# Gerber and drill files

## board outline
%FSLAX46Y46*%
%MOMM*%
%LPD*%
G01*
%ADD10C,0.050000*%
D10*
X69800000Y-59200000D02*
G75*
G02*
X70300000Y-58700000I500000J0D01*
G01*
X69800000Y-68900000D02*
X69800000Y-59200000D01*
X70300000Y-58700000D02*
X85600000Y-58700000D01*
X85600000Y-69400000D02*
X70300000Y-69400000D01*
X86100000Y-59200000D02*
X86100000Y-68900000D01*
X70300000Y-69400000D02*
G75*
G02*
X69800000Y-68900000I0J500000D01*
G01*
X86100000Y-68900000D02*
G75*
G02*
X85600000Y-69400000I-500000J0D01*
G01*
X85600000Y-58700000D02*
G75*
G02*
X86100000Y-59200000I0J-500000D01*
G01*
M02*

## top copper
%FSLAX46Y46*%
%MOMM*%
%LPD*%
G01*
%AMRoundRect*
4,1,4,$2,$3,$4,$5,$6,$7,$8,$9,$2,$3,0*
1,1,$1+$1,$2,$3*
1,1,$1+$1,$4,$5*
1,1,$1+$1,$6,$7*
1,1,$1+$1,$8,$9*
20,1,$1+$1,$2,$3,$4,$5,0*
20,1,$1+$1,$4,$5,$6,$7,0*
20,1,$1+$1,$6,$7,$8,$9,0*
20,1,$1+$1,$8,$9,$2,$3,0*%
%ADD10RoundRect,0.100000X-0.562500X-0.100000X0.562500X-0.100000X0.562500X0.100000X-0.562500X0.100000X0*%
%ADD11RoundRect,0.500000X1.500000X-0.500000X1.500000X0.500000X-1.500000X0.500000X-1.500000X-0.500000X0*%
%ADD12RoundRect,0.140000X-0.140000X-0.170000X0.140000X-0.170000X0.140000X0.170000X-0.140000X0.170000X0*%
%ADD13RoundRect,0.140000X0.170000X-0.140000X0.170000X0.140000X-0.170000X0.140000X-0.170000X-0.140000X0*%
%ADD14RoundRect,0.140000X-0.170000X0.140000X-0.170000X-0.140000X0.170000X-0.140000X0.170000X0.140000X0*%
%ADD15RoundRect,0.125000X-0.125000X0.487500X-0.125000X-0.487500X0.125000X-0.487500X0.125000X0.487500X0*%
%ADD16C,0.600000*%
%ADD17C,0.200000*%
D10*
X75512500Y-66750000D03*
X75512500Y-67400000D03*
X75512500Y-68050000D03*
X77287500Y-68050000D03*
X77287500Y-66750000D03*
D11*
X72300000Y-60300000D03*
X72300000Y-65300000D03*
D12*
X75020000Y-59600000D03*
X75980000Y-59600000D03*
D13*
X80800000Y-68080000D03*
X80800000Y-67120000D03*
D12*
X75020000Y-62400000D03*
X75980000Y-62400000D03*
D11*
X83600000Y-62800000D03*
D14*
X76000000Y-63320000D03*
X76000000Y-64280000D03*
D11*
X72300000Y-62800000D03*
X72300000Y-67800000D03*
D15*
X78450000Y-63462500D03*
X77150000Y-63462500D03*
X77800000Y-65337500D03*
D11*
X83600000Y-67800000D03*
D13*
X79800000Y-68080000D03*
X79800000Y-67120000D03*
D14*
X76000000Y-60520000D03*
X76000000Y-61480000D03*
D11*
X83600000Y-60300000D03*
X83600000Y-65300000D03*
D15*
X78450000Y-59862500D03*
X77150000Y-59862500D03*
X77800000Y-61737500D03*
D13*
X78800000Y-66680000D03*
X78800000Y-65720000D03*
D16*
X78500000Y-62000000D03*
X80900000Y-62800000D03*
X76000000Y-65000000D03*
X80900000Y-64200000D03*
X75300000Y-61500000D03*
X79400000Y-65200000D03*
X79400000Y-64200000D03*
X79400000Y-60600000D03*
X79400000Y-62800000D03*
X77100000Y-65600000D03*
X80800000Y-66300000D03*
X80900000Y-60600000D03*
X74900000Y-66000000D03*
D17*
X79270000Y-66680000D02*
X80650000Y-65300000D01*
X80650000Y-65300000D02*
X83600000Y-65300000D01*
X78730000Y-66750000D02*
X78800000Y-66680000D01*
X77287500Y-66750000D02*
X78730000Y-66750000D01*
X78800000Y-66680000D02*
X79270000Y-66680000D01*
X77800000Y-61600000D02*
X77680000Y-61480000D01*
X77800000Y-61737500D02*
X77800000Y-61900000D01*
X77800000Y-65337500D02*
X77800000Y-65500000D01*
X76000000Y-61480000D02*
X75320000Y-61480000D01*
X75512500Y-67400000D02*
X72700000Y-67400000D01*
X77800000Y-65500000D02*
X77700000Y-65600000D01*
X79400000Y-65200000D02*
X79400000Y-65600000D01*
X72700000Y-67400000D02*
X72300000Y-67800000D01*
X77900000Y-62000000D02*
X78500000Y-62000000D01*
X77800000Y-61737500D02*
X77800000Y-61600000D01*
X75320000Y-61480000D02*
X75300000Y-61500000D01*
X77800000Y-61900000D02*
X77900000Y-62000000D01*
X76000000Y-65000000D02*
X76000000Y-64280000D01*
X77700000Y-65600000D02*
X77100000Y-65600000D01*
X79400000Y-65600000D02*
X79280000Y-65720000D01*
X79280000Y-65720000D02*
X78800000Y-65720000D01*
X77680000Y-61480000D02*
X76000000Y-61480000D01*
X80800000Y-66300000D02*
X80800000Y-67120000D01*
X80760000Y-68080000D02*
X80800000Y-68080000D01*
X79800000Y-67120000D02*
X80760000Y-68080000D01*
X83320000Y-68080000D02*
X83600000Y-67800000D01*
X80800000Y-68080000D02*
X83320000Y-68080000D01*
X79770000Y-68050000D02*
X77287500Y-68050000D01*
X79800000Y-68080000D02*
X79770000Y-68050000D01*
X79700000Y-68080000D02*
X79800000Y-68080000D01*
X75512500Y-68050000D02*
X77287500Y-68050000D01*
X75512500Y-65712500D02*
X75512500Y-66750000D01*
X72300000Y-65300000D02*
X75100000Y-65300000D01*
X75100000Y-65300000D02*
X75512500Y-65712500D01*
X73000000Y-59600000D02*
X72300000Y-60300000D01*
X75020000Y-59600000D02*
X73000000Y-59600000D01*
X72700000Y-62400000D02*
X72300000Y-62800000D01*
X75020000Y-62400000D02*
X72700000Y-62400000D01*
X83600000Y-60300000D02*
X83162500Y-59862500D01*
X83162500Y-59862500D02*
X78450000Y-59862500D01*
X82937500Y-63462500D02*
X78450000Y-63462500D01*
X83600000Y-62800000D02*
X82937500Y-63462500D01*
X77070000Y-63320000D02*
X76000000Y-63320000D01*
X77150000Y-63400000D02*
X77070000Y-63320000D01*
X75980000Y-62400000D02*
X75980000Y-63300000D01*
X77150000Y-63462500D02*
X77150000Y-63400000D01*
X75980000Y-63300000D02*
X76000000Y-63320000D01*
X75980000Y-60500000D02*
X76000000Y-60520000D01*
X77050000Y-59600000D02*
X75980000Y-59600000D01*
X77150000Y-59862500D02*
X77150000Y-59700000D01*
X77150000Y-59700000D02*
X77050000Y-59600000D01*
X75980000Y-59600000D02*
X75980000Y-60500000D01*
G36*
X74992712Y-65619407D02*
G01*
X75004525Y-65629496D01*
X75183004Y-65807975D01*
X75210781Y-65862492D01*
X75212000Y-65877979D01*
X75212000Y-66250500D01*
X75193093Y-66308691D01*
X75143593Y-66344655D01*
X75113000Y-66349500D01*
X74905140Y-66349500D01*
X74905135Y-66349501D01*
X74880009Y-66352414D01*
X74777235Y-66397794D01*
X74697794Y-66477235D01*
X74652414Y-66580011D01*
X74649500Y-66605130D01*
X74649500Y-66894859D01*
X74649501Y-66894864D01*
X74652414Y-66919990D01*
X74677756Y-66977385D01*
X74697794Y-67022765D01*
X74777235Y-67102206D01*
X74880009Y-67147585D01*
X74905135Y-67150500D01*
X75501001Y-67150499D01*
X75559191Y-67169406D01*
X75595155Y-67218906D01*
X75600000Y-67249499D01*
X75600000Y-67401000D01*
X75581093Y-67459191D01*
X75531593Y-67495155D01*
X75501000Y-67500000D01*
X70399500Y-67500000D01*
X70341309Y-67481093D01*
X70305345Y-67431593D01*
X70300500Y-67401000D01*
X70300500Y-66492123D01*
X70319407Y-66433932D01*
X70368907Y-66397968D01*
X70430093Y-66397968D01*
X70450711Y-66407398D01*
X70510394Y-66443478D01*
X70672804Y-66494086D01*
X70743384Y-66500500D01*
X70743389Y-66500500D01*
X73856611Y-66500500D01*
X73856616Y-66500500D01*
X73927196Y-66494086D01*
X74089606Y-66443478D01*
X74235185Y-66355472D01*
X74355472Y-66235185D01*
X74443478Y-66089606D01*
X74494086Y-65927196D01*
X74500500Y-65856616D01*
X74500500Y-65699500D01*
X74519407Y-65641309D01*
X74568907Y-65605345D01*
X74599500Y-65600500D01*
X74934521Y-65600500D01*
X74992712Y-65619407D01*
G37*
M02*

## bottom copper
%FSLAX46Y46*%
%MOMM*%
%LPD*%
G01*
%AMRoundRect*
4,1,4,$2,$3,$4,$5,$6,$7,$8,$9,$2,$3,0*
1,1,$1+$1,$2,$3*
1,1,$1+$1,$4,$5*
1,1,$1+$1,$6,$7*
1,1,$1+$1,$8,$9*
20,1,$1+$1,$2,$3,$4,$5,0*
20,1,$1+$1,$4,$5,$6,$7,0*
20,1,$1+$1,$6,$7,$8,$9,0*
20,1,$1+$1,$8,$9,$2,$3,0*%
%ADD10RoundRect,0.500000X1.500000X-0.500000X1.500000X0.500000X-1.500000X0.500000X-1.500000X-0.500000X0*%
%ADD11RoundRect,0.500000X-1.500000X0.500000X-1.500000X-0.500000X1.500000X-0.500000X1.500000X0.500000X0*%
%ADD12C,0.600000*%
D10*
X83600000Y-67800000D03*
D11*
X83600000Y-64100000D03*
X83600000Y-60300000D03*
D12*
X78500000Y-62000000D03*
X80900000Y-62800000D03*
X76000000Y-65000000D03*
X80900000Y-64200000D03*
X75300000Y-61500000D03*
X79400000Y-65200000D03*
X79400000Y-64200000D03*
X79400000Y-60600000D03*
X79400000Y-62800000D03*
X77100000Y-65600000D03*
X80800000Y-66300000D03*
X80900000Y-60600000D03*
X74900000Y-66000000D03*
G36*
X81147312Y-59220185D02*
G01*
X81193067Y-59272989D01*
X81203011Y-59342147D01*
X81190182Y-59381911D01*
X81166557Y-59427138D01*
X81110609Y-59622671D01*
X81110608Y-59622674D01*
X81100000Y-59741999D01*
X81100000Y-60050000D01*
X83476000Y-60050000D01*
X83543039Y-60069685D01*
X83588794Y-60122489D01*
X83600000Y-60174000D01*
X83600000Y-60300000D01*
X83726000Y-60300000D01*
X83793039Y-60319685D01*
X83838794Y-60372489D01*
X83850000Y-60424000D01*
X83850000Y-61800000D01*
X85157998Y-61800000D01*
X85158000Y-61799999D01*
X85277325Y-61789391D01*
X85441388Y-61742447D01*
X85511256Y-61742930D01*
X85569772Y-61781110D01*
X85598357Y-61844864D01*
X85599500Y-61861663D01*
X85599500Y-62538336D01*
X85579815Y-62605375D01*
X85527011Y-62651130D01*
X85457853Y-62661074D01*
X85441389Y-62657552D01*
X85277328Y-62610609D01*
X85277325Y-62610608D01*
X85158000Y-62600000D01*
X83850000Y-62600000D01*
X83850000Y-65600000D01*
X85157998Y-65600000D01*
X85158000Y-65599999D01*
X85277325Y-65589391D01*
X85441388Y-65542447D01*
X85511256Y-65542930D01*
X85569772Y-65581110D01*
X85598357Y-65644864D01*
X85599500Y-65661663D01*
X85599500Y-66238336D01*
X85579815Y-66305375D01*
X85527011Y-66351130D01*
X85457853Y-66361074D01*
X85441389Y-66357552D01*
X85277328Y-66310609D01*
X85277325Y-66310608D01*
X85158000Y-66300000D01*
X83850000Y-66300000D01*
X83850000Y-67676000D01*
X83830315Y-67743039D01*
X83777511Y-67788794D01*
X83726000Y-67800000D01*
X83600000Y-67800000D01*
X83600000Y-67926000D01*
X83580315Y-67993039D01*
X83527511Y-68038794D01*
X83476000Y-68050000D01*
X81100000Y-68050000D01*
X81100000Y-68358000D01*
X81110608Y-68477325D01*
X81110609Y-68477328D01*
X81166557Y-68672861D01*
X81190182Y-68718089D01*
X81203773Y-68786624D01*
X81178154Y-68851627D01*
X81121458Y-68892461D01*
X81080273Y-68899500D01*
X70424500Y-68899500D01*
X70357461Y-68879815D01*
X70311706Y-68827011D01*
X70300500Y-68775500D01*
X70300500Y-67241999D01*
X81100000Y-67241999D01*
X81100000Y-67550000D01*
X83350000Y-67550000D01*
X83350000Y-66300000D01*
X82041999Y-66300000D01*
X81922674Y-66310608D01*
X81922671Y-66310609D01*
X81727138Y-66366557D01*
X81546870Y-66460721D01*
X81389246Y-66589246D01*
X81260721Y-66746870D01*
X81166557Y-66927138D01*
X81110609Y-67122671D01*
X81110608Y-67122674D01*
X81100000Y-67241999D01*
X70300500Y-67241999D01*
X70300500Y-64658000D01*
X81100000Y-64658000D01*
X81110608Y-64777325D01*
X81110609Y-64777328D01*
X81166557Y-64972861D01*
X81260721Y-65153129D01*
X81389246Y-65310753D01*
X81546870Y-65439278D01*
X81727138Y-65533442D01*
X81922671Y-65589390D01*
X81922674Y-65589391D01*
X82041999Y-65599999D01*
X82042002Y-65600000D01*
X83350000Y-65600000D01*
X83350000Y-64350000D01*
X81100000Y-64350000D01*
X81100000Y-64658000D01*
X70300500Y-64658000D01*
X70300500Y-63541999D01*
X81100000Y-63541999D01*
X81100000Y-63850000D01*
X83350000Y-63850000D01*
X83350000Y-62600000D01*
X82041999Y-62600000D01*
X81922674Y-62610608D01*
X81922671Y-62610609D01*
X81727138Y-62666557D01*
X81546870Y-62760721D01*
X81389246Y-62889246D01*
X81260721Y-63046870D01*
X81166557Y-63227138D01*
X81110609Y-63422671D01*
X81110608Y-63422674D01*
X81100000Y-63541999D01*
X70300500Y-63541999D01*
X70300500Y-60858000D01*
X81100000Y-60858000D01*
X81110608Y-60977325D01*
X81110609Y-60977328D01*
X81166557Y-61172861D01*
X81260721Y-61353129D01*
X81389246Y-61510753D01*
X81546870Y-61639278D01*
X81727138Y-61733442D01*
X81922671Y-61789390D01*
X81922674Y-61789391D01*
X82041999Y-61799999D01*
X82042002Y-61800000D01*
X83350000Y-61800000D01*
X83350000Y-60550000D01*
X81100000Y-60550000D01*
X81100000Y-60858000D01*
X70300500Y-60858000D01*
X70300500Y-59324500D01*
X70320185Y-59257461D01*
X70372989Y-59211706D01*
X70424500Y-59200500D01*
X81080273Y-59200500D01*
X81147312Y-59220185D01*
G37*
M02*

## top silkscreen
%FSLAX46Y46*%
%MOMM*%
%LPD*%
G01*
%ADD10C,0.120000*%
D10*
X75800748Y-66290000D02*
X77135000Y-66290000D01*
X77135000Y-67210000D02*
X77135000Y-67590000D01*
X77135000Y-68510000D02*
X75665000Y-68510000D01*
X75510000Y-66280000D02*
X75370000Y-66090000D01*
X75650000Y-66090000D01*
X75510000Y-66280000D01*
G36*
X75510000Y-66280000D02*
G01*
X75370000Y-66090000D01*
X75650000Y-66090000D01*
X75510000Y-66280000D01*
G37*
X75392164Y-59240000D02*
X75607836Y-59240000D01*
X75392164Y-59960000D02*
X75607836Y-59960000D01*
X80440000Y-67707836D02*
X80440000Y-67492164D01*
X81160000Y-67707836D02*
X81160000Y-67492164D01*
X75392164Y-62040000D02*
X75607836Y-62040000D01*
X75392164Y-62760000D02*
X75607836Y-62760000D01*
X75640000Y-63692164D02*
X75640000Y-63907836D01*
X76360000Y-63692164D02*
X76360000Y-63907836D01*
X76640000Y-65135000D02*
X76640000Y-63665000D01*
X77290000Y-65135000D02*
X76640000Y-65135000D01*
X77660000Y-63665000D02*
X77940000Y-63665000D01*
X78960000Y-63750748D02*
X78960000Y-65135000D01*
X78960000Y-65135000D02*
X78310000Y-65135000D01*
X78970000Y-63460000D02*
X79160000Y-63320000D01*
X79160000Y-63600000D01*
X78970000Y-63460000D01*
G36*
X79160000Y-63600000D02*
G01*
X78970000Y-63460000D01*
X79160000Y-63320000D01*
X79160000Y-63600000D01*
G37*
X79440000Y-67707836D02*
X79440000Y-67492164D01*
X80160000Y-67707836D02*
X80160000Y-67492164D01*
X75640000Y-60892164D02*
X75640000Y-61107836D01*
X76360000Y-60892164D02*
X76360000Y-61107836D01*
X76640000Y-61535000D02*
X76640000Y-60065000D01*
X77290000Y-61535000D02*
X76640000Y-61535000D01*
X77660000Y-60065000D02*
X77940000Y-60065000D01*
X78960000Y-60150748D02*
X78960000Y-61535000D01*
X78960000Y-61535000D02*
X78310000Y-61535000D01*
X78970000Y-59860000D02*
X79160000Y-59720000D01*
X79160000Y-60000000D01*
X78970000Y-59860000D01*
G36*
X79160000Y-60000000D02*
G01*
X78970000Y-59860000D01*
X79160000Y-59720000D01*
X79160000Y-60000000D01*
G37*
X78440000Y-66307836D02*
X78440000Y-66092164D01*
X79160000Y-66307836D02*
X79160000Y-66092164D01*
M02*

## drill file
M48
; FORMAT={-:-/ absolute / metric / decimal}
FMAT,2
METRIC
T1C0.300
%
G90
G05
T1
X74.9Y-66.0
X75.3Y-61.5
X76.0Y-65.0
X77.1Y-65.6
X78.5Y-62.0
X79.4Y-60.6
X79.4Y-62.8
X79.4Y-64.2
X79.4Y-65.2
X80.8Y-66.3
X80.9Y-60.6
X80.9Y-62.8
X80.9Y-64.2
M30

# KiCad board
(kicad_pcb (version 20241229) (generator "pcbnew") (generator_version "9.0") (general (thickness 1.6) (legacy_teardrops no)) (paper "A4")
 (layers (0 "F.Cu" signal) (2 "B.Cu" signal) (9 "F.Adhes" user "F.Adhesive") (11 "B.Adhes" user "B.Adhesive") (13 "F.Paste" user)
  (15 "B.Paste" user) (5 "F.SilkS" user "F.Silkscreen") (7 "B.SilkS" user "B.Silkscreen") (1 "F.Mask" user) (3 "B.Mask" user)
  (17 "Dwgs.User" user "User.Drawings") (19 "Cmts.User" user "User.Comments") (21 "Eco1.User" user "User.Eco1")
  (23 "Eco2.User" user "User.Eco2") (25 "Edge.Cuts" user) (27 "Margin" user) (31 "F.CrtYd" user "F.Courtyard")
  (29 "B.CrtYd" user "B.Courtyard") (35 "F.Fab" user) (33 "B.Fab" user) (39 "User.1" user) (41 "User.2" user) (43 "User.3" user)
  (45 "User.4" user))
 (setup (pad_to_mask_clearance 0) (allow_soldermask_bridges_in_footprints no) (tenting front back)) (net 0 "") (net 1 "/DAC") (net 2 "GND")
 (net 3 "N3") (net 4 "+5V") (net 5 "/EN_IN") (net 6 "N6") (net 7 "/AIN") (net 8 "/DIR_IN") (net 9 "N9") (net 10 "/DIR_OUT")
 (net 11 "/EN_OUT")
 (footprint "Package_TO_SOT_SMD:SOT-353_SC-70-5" (layer "F.Cu") (at 76.4 67.4)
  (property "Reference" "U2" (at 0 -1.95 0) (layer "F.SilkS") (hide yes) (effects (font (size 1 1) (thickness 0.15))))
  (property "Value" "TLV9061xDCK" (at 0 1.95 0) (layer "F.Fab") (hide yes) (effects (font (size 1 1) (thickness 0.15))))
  (fp_line (start -0.599252 -1.11) (end 0.735 -1.11) (stroke (width 0.12) (type solid)) (layer "F.SilkS"))
  (fp_line (start 0.735 -0.19) (end 0.735 0.19) (stroke (width 0.12) (type solid)) (layer "F.SilkS"))
  (fp_line (start 0.735 1.11) (end -0.735 1.11) (stroke (width 0.12) (type solid)) (layer "F.SilkS"))
  (fp_poly (pts (xy -0.89 -1.12) (xy -1.03 -1.31) (xy -0.75 -1.31)) (stroke (width 0.12) (type solid)) (fill yes) (layer "F.SilkS"))
  (pad "1" smd roundrect (at -0.8875 -0.65) (size 1.325 0.4) (layers "F.Cu" "F.Mask" "F.Paste") (roundrect_rratio 0.25) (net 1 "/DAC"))
  (pad "2" smd roundrect (at -0.8875 0) (size 1.325 0.4) (layers "F.Cu" "F.Mask" "F.Paste") (roundrect_rratio 0.25) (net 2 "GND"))
  (pad "3" smd roundrect (at -0.8875 0.65) (size 1.325 0.4) (layers "F.Cu" "F.Mask" "F.Paste") (roundrect_rratio 0.25) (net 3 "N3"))
  (pad "4" smd roundrect (at 0.8875 0.65) (size 1.325 0.4) (layers "F.Cu" "F.Mask" "F.Paste") (roundrect_rratio 0.25) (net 3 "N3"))
  (pad "5" smd roundrect (at 0.8875 -0.65) (size 1.325 0.4) (layers "F.Cu" "F.Mask" "F.Paste") (roundrect_rratio 0.25) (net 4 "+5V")))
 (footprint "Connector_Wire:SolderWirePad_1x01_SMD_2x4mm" (layer "F.Cu") (at 72.3 60.3 90)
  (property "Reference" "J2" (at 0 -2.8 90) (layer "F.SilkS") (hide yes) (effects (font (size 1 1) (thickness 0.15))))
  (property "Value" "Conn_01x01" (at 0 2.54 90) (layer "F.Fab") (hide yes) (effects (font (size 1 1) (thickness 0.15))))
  (pad "1" smd roundrect (at 0 0 90) (size 2 4) (layers "F.Cu" "F.Mask") (roundrect_rratio 0.25) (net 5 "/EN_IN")))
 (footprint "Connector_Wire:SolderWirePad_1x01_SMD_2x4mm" (layer "F.Cu") (at 72.3 65.3 90)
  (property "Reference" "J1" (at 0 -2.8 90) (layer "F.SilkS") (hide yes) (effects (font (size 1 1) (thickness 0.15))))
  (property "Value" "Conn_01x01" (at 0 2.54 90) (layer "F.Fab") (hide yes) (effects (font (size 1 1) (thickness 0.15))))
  (pad "1" smd roundrect (at 0 0 90) (size 2 4) (layers "F.Cu" "F.Mask") (roundrect_rratio 0.25) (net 1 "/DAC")))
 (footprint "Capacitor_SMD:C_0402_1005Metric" (layer "F.Cu") (at 75.5 59.6)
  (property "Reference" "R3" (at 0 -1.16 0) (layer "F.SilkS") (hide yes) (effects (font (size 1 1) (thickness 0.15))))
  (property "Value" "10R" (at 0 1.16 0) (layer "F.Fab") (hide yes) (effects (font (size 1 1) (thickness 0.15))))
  (fp_line (start -0.107836 -0.36) (end 0.107836 -0.36) (stroke (width 0.12) (type solid)) (layer "F.SilkS"))
  (fp_line (start -0.107836 0.36) (end 0.107836 0.36) (stroke (width 0.12) (type solid)) (layer "F.SilkS"))
  (pad "1" smd roundrect (at -0.48 0) (size 0.56 0.62) (layers "F.Cu" "F.Mask" "F.Paste") (roundrect_rratio 0.25) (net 5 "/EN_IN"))
  (pad "2" smd roundrect (at 0.48 0) (size 0.56 0.62) (layers "F.Cu" "F.Mask" "F.Paste") (roundrect_rratio 0.25) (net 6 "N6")))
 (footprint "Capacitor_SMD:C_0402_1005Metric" (layer "F.Cu") (at 80.8 67.6 90)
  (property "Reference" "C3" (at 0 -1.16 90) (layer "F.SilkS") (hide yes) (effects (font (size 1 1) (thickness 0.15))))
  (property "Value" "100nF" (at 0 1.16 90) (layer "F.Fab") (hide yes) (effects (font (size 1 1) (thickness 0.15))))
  (fp_line (start -0.107836 -0.36) (end 0.107836 -0.36) (stroke (width 0.12) (type solid)) (layer "F.SilkS"))
  (fp_line (start -0.107836 0.36) (end 0.107836 0.36) (stroke (width 0.12) (type solid)) (layer "F.SilkS"))
  (pad "1" smd roundrect (at -0.48 0 90) (size 0.56 0.62) (layers "F.Cu" "F.Mask" "F.Paste") (roundrect_rratio 0.25) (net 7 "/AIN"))
  (pad "2" smd roundrect (at 0.48 0 90) (size 0.56 0.62) (layers "F.Cu" "F.Mask" "F.Paste") (roundrect_rratio 0.25) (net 2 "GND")))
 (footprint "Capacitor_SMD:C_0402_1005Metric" (layer "F.Cu") (at 75.5 62.4)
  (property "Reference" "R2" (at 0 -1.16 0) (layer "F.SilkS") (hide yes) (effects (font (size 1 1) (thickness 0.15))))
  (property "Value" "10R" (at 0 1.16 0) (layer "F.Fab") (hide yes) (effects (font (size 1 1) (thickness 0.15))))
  (fp_line (start -0.107836 -0.36) (end 0.107836 -0.36) (stroke (width 0.12) (type solid)) (layer "F.SilkS"))
  (fp_line (start -0.107836 0.36) (end 0.107836 0.36) (stroke (width 0.12) (type solid)) (layer "F.SilkS"))
  (pad "1" smd roundrect (at -0.48 0) (size 0.56 0.62) (layers "F.Cu" "F.Mask" "F.Paste") (roundrect_rratio 0.25) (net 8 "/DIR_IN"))
  (pad "2" smd roundrect (at 0.48 0) (size 0.56 0.62) (layers "F.Cu" "F.Mask" "F.Paste") (roundrect_rratio 0.25) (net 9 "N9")))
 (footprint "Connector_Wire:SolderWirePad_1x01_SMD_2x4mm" (layer "F.Cu") (at 83.6 62.8 90)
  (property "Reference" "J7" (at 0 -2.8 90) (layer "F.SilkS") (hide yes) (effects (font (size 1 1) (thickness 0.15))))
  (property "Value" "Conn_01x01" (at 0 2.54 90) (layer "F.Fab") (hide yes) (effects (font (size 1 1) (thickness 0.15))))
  (pad "1" smd roundrect (at 0 0 90) (size 2 4) (layers "F.Cu" "F.Mask") (roundrect_rratio 0.25) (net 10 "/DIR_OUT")))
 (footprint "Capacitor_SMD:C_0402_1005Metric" (layer "F.Cu") (at 76 63.8 -90)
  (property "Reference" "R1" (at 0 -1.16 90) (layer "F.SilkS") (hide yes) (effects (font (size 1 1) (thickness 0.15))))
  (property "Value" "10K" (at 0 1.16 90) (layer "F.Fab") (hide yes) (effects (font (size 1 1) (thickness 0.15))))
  (fp_line (start -0.107836 0.36) (end 0.107836 0.36) (stroke (width 0.12) (type solid)) (layer "F.SilkS"))
  (fp_line (start -0.107836 -0.36) (end 0.107836 -0.36) (stroke (width 0.12) (type solid)) (layer "F.SilkS"))
  (pad "1" smd roundrect (at -0.48 0 270) (size 0.56 0.62) (layers "F.Cu" "F.Mask" "F.Paste") (roundrect_rratio 0.25) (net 9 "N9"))
  (pad "2" smd roundrect (at 0.48 0 270) (size 0.56 0.62) (layers "F.Cu" "F.Mask" "F.Paste") (roundrect_rratio 0.25) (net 2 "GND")))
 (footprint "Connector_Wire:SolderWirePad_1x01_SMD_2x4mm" (layer "F.Cu") (at 72.3 62.8 90)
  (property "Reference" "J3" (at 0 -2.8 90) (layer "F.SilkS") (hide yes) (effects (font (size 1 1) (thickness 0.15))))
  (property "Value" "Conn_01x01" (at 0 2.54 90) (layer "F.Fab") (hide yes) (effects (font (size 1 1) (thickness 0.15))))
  (pad "1" smd roundrect (at 0 0 90) (size 2 4) (layers "F.Cu" "F.Mask") (roundrect_rratio 0.25) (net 8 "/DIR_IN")))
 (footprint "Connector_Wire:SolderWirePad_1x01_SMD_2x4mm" (layer "F.Cu") (at 72.3 67.8 90)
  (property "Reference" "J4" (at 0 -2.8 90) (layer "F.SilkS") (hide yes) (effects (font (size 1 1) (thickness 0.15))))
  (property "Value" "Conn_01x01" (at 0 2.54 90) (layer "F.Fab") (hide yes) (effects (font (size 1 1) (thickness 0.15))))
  (pad "1" smd roundrect (at 0 0 90) (size 2 4) (layers "F.Cu" "F.Mask") (roundrect_rratio 0.25) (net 2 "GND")))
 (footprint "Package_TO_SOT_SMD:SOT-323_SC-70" (layer "F.Cu") (at 77.8 64.4 -90)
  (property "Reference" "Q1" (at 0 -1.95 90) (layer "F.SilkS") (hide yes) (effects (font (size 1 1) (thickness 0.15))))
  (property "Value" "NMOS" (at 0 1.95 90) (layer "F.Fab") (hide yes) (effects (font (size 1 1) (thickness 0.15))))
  (fp_line (start 0.735 1.16) (end -0.735 1.16) (stroke (width 0.12) (type solid)) (layer "F.SilkS"))
  (fp_line (start 0.735 0.51) (end 0.735 1.16) (stroke (width 0.12) (type solid)) (layer "F.SilkS"))
  (fp_line (start -0.735 0.14) (end -0.735 -0.14) (stroke (width 0.12) (type solid)) (layer "F.SilkS"))
  (fp_line (start -0.649252 -1.16) (end 0.735 -1.16) (stroke (width 0.12) (type solid)) (layer "F.SilkS"))
  (fp_line (start 0.735 -1.16) (end 0.735 -0.51) (stroke (width 0.12) (type solid)) (layer "F.SilkS"))
  (fp_poly (pts (xy -0.94 -1.17) (xy -1.08 -1.36) (xy -0.8 -1.36)) (stroke (width 0.12) (type solid)) (fill yes) (layer "F.SilkS"))
  (pad "1" smd roundrect (at -0.9375 -0.65 270) (size 1.225 0.5) (layers "F.Cu" "F.Mask" "F.Paste") (roundrect_rratio 0.25)
   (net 10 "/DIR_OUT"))
  (pad "2" smd roundrect (at -0.9375 0.65 270) (size 1.225 0.5) (layers "F.Cu" "F.Mask" "F.Paste") (roundrect_rratio 0.25) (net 9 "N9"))
  (pad "3" smd roundrect (at 0.9375 0 270) (size 1.225 0.5) (layers "F.Cu" "F.Mask" "F.Paste") (roundrect_rratio 0.25) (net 2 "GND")))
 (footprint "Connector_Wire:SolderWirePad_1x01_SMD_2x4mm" (layer "F.Cu") (at 83.6 67.8 90)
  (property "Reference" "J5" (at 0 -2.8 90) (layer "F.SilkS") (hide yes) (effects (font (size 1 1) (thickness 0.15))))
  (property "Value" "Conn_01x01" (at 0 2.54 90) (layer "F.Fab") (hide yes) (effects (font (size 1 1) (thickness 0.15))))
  (pad "1" smd roundrect (at 0 0 90) (size 2 4) (layers "F.Cu" "F.Mask") (roundrect_rratio 0.25) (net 7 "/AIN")))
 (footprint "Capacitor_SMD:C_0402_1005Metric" (layer "F.Cu") (at 79.8 67.6 90)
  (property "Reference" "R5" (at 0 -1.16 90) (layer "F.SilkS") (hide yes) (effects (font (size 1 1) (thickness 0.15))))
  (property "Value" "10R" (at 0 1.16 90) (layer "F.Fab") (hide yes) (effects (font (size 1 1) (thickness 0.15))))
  (fp_line (start -0.107836 -0.36) (end 0.107836 -0.36) (stroke (width 0.12) (type solid)) (layer "F.SilkS"))
  (fp_line (start -0.107836 0.36) (end 0.107836 0.36) (stroke (width 0.12) (type solid)) (layer "F.SilkS"))
  (pad "1" smd roundrect (at -0.48 0 90) (size 0.56 0.62) (layers "F.Cu" "F.Mask" "F.Paste") (roundrect_rratio 0.25) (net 3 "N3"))
  (pad "2" smd roundrect (at 0.48 0 90) (size 0.56 0.62) (layers "F.Cu" "F.Mask" "F.Paste") (roundrect_rratio 0.25) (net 7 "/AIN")))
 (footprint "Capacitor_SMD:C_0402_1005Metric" (layer "F.Cu") (at 76 61 -90)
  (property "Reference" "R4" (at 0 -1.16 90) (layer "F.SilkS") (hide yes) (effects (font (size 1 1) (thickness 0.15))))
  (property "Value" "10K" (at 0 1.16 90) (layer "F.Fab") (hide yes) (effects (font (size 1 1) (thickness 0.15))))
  (fp_line (start -0.107836 0.36) (end 0.107836 0.36) (stroke (width 0.12) (type solid)) (layer "F.SilkS"))
  (fp_line (start -0.107836 -0.36) (end 0.107836 -0.36) (stroke (width 0.12) (type solid)) (layer "F.SilkS"))
  (pad "1" smd roundrect (at -0.48 0 270) (size 0.56 0.62) (layers "F.Cu" "F.Mask" "F.Paste") (roundrect_rratio 0.25) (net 6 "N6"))
  (pad "2" smd roundrect (at 0.48 0 270) (size 0.56 0.62) (layers "F.Cu" "F.Mask" "F.Paste") (roundrect_rratio 0.25) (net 2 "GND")))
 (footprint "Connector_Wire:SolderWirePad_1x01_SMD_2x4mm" (layer "F.Cu") (at 83.6 60.3 90)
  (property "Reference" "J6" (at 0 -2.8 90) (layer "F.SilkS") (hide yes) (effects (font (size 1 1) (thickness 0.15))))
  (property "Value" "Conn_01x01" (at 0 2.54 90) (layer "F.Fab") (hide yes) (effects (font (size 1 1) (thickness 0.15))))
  (pad "1" smd roundrect (at 0 0 90) (size 2 4) (layers "F.Cu" "F.Mask") (roundrect_rratio 0.25) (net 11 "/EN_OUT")))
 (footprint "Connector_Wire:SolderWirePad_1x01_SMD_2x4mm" (layer "F.Cu") (at 83.6 65.3 90)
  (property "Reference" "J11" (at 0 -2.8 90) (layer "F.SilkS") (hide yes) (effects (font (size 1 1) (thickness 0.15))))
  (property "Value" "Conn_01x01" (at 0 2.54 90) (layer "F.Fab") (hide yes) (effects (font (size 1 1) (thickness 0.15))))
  (pad "1" smd roundrect (at 0 0 90) (size 2 4) (layers "F.Cu" "F.Mask") (roundrect_rratio 0.25) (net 4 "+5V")))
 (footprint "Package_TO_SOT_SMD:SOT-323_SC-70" (layer "F.Cu") (at 77.8 60.8 -90)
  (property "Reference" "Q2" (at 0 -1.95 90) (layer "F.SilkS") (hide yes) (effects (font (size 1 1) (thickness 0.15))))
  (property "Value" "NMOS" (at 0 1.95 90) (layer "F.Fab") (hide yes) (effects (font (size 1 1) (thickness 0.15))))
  (fp_line (start 0.735 1.16) (end -0.735 1.16) (stroke (width 0.12) (type solid)) (layer "F.SilkS"))
  (fp_line (start 0.735 0.51) (end 0.735 1.16) (stroke (width 0.12) (type solid)) (layer "F.SilkS"))
  (fp_line (start -0.735 0.14) (end -0.735 -0.14) (stroke (width 0.12) (type solid)) (layer "F.SilkS"))
  (fp_line (start -0.649252 -1.16) (end 0.735 -1.16) (stroke (width 0.12) (type solid)) (layer "F.SilkS"))
  (fp_line (start 0.735 -1.16) (end 0.735 -0.51) (stroke (width 0.12) (type solid)) (layer "F.SilkS"))
  (fp_poly (pts (xy -0.94 -1.17) (xy -1.08 -1.36) (xy -0.8 -1.36)) (stroke (width 0.12) (type solid)) (fill yes) (layer "F.SilkS"))
  (pad "1" smd roundrect (at -0.9375 -0.65 270) (size 1.225 0.5) (layers "F.Cu" "F.Mask" "F.Paste") (roundrect_rratio 0.25)
   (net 11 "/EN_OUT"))
  (pad "2" smd roundrect (at -0.9375 0.65 270) (size 1.225 0.5) (layers "F.Cu" "F.Mask" "F.Paste") (roundrect_rratio 0.25) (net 6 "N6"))
  (pad "3" smd roundrect (at 0.9375 0 270) (size 1.225 0.5) (layers "F.Cu" "F.Mask" "F.Paste") (roundrect_rratio 0.25) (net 2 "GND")))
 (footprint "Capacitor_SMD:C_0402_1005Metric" (layer "F.Cu") (at 78.8 66.2 90)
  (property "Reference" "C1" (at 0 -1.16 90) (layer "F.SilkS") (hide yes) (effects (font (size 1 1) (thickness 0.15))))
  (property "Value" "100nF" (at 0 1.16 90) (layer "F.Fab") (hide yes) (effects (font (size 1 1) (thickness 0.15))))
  (fp_line (start -0.107836 -0.36) (end 0.107836 -0.36) (stroke (width 0.12) (type solid)) (layer "F.SilkS"))
  (fp_line (start -0.107836 0.36) (end 0.107836 0.36) (stroke (width 0.12) (type solid)) (layer "F.SilkS"))
  (pad "1" smd roundrect (at -0.48 0 90) (size 0.56 0.62) (layers "F.Cu" "F.Mask" "F.Paste") (roundrect_rratio 0.25) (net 4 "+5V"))
  (pad "2" smd roundrect (at 0.48 0 90) (size 0.56 0.62) (layers "F.Cu" "F.Mask" "F.Paste") (roundrect_rratio 0.25) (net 2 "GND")))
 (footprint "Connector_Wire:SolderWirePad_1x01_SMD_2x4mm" (layer "B.Cu") (at 83.6 67.8 90)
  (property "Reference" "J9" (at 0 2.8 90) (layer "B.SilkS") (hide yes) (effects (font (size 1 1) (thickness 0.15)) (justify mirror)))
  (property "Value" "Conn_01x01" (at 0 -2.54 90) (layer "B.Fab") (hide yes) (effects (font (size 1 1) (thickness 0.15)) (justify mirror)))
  (pad "1" smd roundrect (at 0 0 90) (size 2 4) (layers "B.Cu" "B.Mask") (roundrect_rratio 0.25) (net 2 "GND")))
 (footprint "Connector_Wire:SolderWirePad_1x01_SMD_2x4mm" (layer "B.Cu") (at 83.6 64.1 -90)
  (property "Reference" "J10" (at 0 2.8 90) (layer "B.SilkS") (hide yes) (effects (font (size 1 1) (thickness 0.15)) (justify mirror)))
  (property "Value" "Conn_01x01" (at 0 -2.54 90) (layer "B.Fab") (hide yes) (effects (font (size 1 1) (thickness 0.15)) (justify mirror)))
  (pad "1" smd roundrect (at 0 0 270) (size 2 4) (layers "B.Cu" "B.Mask") (roundrect_rratio 0.25) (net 2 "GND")))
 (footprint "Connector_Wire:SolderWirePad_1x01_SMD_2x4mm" (layer "B.Cu") (at 83.6 60.3 -90)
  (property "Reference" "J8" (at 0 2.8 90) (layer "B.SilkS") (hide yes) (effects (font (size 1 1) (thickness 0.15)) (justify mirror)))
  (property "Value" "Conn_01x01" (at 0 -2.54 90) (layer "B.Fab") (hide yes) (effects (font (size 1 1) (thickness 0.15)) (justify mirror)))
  (pad "1" smd roundrect (at 0 0 270) (size 2 4) (layers "B.Cu" "B.Mask") (roundrect_rratio 0.25) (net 2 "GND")))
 (gr_arc (start 69.8 59.2) (mid 69.946447 58.846447) (end 70.3 58.7) (stroke (width 0.05) (type default)) (layer "Edge.Cuts"))
 (gr_line (start 69.8 68.9) (end 69.8 59.2) (stroke (width 0.05) (type default)) (layer "Edge.Cuts"))
 (gr_line (start 70.3 58.7) (end 85.6 58.7) (stroke (width 0.05) (type default)) (layer "Edge.Cuts"))
 (gr_line (start 85.6 69.4) (end 70.3 69.4) (stroke (width 0.05) (type default)) (layer "Edge.Cuts"))
 (gr_line (start 86.1 59.2) (end 86.1 68.9) (stroke (width 0.05) (type default)) (layer "Edge.Cuts"))
 (gr_arc (start 70.3 69.4) (mid 69.946447 69.253553) (end 69.8 68.9) (stroke (width 0.05) (type default)) (layer "Edge.Cuts"))
 (gr_arc (start 86.1 68.9) (mid 85.953553 69.253553) (end 85.6 69.4) (stroke (width 0.05) (type default)) (layer "Edge.Cuts"))
 (gr_arc (start 85.6 58.7) (mid 85.953553 58.846447) (end 86.1 59.2) (stroke (width 0.05) (type default)) (layer "Edge.Cuts"))
 (segment (start 79.27 66.68) (end 80.65 65.3) (width 0.2) (layer "F.Cu") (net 4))
 (segment (start 80.65 65.3) (end 83.6 65.3) (width 0.2) (layer "F.Cu") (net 4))
 (segment (start 78.73 66.75) (end 78.8 66.68) (width 0.2) (layer "F.Cu") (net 4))
 (segment (start 77.2875 66.75) (end 78.73 66.75) (width 0.2) (layer "F.Cu") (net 4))
 (segment (start 78.8 66.68) (end 79.27 66.68) (width 0.2) (layer "F.Cu") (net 4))
 (segment (start 77.8 61.6) (end 77.68 61.48) (width 0.2) (layer "F.Cu") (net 2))
 (segment (start 77.8 61.7375) (end 77.8 61.9) (width 0.2) (layer "F.Cu") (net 2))
 (segment (start 77.8 65.3375) (end 77.8 65.5) (width 0.2) (layer "F.Cu") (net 2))
 (segment (start 76 61.48) (end 75.32 61.48) (width 0.2) (layer "F.Cu") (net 2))
 (segment (start 75.5125 67.4) (end 72.7 67.4) (width 0.2) (layer "F.Cu") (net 2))
 (segment (start 77.8 65.5) (end 77.7 65.6) (width 0.2) (layer "F.Cu") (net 2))
 (segment (start 79.4 65.2) (end 79.4 65.6) (width 0.2) (layer "F.Cu") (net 2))
 (segment (start 72.7 67.4) (end 72.3 67.8) (width 0.2) (layer "F.Cu") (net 2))
 (segment (start 77.9 62) (end 78.5 62) (width 0.2) (layer "F.Cu") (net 2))
 (segment (start 77.8 61.7375) (end 77.8 61.6) (width 0.2) (layer "F.Cu") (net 2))
 (segment (start 75.32 61.48) (end 75.3 61.5) (width 0.2) (layer "F.Cu") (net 2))
 (segment (start 77.8 61.9) (end 77.9 62) (width 0.2) (layer "F.Cu") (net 2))
 (segment (start 76 65) (end 76 64.28) (width 0.2) (layer "F.Cu") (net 2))
 (segment (start 77.7 65.6) (end 77.1 65.6) (width 0.2) (layer "F.Cu") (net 2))
 (segment (start 79.4 65.6) (end 79.28 65.72) (width 0.2) (layer "F.Cu") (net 2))
 (segment (start 79.28 65.72) (end 78.8 65.72) (width 0.2) (layer "F.Cu") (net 2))
 (segment (start 77.68 61.48) (end 76 61.48) (width 0.2) (layer "F.Cu") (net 2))
 (segment (start 80.8 66.3) (end 80.8 67.12) (width 0.2) (layer "F.Cu") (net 2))
 (via (at 78.5 62) (size 0.6) (drill 0.3) (layers "F.Cu" "B.Cu") (free yes) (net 2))
 (via (at 80.9 62.8) (size 0.6) (drill 0.3) (layers "F.Cu" "B.Cu") (free yes) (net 2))
 (via (at 76 65) (size 0.6) (drill 0.3) (layers "F.Cu" "B.Cu") (free yes) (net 2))
 (via (at 80.9 64.2) (size 0.6) (drill 0.3) (layers "F.Cu" "B.Cu") (free yes) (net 2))
 (via (at 75.3 61.5) (size 0.6) (drill 0.3) (layers "F.Cu" "B.Cu") (free yes) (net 2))
 (via (at 79.4 65.2) (size 0.6) (drill 0.3) (layers "F.Cu" "B.Cu") (free yes) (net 2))
 (via (at 79.4 64.2) (size 0.6) (drill 0.3) (layers "F.Cu" "B.Cu") (free yes) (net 2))
 (via (at 79.4 60.6) (size 0.6) (drill 0.3) (layers "F.Cu" "B.Cu") (free yes) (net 2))
 (via (at 79.4 62.8) (size 0.6) (drill 0.3) (layers "F.Cu" "B.Cu") (free yes) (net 2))
 (via (at 77.1 65.6) (size 0.6) (drill 0.3) (layers "F.Cu" "B.Cu") (free yes) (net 2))
 (via (at 80.8 66.3) (size 0.6) (drill 0.3) (layers "F.Cu" "B.Cu") (free yes) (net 2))
 (via (at 80.9 60.6) (size 0.6) (drill 0.3) (layers "F.Cu" "B.Cu") (free yes) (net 2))
 (via (at 74.9 66) (size 0.6) (drill 0.3) (layers "F.Cu" "B.Cu") (free yes) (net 2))
 (segment (start 80.76 68.08) (end 80.8 68.08) (width 0.2) (layer "F.Cu") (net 7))
 (segment (start 79.8 67.12) (end 80.76 68.08) (width 0.2) (layer "F.Cu") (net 7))
 (segment (start 83.32 68.08) (end 83.6 67.8) (width 0.2) (layer "F.Cu") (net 7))
 (segment (start 80.8 68.08) (end 83.32 68.08) (width 0.2) (layer "F.Cu") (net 7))
 (segment (start 79.77 68.05) (end 77.2875 68.05) (width 0.2) (layer "F.Cu") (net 3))
 (segment (start 79.8 68.08) (end 79.77 68.05) (width 0.2) (layer "F.Cu") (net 3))
 (segment (start 79.7 68.08) (end 79.8 68.08) (width 0.2) (layer "F.Cu") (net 3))
 (segment (start 75.5125 68.05) (end 77.2875 68.05) (width 0.2) (layer "F.Cu") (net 3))
 (segment (start 75.5125 65.7125) (end 75.5125 66.75) (width 0.2) (layer "F.Cu") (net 1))
 (segment (start 72.3 65.3) (end 75.1 65.3) (width 0.2) (layer "F.Cu") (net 1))
 (segment (start 75.1 65.3) (end 75.5125 65.7125) (width 0.2) (layer "F.Cu") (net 1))
 (segment (start 73 59.6) (end 72.3 60.3) (width 0.2) (layer "F.Cu") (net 5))
 (segment (start 75.02 59.6) (end 73 59.6) (width 0.2) (layer "F.Cu") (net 5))
 (segment (start 72.7 62.4) (end 72.3 62.8) (width 0.2) (layer "F.Cu") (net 8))
 (segment (start 75.02 62.4) (end 72.7 62.4) (width 0.2) (layer "F.Cu") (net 8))
 (segment (start 83.6 60.3) (end 83.1625 59.8625) (width 0.2) (layer "F.Cu") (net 11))
 (segment (start 83.1625 59.8625) (end 78.45 59.8625) (width 0.2) (layer "F.Cu") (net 11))
 (segment (start 82.9375 63.4625) (end 78.45 63.4625) (width 0.2) (layer "F.Cu") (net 10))
 (segment (start 83.6 62.8) (end 82.9375 63.4625) (width 0.2) (layer "F.Cu") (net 10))
 (segment (start 77.07 63.32) (end 76 63.32) (width 0.2) (layer "F.Cu") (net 9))
 (segment (start 77.15 63.4) (end 77.07 63.32) (width 0.2) (layer "F.Cu") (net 9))
 (segment (start 75.98 62.4) (end 75.98 63.3) (width 0.2) (layer "F.Cu") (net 9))
 (segment (start 77.15 63.4625) (end 77.15 63.4) (width 0.2) (layer "F.Cu") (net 9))
 (segment (start 75.98 63.3) (end 76 63.32) (width 0.2) (layer "F.Cu") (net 9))
 (segment (start 75.98 60.5) (end 76 60.52) (width 0.2) (layer "F.Cu") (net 6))
 (segment (start 77.05 59.6) (end 75.98 59.6) (width 0.2) (layer "F.Cu") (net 6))
 (segment (start 77.15 59.8625) (end 77.15 59.7) (width 0.2) (layer "F.Cu") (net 6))
 (segment (start 77.15 59.7) (end 77.05 59.6) (width 0.2) (layer "F.Cu") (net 6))
 (segment (start 75.98 59.6) (end 75.98 60.5) (width 0.2) (layer "F.Cu") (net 6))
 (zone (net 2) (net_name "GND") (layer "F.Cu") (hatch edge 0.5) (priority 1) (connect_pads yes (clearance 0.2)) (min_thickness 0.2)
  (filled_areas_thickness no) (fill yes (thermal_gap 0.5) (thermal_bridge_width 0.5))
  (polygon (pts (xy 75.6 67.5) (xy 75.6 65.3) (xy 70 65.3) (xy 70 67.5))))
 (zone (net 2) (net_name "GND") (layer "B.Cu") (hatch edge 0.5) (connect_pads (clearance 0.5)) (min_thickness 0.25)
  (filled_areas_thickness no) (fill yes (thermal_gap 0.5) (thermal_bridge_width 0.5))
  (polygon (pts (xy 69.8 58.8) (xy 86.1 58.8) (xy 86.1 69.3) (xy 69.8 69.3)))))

